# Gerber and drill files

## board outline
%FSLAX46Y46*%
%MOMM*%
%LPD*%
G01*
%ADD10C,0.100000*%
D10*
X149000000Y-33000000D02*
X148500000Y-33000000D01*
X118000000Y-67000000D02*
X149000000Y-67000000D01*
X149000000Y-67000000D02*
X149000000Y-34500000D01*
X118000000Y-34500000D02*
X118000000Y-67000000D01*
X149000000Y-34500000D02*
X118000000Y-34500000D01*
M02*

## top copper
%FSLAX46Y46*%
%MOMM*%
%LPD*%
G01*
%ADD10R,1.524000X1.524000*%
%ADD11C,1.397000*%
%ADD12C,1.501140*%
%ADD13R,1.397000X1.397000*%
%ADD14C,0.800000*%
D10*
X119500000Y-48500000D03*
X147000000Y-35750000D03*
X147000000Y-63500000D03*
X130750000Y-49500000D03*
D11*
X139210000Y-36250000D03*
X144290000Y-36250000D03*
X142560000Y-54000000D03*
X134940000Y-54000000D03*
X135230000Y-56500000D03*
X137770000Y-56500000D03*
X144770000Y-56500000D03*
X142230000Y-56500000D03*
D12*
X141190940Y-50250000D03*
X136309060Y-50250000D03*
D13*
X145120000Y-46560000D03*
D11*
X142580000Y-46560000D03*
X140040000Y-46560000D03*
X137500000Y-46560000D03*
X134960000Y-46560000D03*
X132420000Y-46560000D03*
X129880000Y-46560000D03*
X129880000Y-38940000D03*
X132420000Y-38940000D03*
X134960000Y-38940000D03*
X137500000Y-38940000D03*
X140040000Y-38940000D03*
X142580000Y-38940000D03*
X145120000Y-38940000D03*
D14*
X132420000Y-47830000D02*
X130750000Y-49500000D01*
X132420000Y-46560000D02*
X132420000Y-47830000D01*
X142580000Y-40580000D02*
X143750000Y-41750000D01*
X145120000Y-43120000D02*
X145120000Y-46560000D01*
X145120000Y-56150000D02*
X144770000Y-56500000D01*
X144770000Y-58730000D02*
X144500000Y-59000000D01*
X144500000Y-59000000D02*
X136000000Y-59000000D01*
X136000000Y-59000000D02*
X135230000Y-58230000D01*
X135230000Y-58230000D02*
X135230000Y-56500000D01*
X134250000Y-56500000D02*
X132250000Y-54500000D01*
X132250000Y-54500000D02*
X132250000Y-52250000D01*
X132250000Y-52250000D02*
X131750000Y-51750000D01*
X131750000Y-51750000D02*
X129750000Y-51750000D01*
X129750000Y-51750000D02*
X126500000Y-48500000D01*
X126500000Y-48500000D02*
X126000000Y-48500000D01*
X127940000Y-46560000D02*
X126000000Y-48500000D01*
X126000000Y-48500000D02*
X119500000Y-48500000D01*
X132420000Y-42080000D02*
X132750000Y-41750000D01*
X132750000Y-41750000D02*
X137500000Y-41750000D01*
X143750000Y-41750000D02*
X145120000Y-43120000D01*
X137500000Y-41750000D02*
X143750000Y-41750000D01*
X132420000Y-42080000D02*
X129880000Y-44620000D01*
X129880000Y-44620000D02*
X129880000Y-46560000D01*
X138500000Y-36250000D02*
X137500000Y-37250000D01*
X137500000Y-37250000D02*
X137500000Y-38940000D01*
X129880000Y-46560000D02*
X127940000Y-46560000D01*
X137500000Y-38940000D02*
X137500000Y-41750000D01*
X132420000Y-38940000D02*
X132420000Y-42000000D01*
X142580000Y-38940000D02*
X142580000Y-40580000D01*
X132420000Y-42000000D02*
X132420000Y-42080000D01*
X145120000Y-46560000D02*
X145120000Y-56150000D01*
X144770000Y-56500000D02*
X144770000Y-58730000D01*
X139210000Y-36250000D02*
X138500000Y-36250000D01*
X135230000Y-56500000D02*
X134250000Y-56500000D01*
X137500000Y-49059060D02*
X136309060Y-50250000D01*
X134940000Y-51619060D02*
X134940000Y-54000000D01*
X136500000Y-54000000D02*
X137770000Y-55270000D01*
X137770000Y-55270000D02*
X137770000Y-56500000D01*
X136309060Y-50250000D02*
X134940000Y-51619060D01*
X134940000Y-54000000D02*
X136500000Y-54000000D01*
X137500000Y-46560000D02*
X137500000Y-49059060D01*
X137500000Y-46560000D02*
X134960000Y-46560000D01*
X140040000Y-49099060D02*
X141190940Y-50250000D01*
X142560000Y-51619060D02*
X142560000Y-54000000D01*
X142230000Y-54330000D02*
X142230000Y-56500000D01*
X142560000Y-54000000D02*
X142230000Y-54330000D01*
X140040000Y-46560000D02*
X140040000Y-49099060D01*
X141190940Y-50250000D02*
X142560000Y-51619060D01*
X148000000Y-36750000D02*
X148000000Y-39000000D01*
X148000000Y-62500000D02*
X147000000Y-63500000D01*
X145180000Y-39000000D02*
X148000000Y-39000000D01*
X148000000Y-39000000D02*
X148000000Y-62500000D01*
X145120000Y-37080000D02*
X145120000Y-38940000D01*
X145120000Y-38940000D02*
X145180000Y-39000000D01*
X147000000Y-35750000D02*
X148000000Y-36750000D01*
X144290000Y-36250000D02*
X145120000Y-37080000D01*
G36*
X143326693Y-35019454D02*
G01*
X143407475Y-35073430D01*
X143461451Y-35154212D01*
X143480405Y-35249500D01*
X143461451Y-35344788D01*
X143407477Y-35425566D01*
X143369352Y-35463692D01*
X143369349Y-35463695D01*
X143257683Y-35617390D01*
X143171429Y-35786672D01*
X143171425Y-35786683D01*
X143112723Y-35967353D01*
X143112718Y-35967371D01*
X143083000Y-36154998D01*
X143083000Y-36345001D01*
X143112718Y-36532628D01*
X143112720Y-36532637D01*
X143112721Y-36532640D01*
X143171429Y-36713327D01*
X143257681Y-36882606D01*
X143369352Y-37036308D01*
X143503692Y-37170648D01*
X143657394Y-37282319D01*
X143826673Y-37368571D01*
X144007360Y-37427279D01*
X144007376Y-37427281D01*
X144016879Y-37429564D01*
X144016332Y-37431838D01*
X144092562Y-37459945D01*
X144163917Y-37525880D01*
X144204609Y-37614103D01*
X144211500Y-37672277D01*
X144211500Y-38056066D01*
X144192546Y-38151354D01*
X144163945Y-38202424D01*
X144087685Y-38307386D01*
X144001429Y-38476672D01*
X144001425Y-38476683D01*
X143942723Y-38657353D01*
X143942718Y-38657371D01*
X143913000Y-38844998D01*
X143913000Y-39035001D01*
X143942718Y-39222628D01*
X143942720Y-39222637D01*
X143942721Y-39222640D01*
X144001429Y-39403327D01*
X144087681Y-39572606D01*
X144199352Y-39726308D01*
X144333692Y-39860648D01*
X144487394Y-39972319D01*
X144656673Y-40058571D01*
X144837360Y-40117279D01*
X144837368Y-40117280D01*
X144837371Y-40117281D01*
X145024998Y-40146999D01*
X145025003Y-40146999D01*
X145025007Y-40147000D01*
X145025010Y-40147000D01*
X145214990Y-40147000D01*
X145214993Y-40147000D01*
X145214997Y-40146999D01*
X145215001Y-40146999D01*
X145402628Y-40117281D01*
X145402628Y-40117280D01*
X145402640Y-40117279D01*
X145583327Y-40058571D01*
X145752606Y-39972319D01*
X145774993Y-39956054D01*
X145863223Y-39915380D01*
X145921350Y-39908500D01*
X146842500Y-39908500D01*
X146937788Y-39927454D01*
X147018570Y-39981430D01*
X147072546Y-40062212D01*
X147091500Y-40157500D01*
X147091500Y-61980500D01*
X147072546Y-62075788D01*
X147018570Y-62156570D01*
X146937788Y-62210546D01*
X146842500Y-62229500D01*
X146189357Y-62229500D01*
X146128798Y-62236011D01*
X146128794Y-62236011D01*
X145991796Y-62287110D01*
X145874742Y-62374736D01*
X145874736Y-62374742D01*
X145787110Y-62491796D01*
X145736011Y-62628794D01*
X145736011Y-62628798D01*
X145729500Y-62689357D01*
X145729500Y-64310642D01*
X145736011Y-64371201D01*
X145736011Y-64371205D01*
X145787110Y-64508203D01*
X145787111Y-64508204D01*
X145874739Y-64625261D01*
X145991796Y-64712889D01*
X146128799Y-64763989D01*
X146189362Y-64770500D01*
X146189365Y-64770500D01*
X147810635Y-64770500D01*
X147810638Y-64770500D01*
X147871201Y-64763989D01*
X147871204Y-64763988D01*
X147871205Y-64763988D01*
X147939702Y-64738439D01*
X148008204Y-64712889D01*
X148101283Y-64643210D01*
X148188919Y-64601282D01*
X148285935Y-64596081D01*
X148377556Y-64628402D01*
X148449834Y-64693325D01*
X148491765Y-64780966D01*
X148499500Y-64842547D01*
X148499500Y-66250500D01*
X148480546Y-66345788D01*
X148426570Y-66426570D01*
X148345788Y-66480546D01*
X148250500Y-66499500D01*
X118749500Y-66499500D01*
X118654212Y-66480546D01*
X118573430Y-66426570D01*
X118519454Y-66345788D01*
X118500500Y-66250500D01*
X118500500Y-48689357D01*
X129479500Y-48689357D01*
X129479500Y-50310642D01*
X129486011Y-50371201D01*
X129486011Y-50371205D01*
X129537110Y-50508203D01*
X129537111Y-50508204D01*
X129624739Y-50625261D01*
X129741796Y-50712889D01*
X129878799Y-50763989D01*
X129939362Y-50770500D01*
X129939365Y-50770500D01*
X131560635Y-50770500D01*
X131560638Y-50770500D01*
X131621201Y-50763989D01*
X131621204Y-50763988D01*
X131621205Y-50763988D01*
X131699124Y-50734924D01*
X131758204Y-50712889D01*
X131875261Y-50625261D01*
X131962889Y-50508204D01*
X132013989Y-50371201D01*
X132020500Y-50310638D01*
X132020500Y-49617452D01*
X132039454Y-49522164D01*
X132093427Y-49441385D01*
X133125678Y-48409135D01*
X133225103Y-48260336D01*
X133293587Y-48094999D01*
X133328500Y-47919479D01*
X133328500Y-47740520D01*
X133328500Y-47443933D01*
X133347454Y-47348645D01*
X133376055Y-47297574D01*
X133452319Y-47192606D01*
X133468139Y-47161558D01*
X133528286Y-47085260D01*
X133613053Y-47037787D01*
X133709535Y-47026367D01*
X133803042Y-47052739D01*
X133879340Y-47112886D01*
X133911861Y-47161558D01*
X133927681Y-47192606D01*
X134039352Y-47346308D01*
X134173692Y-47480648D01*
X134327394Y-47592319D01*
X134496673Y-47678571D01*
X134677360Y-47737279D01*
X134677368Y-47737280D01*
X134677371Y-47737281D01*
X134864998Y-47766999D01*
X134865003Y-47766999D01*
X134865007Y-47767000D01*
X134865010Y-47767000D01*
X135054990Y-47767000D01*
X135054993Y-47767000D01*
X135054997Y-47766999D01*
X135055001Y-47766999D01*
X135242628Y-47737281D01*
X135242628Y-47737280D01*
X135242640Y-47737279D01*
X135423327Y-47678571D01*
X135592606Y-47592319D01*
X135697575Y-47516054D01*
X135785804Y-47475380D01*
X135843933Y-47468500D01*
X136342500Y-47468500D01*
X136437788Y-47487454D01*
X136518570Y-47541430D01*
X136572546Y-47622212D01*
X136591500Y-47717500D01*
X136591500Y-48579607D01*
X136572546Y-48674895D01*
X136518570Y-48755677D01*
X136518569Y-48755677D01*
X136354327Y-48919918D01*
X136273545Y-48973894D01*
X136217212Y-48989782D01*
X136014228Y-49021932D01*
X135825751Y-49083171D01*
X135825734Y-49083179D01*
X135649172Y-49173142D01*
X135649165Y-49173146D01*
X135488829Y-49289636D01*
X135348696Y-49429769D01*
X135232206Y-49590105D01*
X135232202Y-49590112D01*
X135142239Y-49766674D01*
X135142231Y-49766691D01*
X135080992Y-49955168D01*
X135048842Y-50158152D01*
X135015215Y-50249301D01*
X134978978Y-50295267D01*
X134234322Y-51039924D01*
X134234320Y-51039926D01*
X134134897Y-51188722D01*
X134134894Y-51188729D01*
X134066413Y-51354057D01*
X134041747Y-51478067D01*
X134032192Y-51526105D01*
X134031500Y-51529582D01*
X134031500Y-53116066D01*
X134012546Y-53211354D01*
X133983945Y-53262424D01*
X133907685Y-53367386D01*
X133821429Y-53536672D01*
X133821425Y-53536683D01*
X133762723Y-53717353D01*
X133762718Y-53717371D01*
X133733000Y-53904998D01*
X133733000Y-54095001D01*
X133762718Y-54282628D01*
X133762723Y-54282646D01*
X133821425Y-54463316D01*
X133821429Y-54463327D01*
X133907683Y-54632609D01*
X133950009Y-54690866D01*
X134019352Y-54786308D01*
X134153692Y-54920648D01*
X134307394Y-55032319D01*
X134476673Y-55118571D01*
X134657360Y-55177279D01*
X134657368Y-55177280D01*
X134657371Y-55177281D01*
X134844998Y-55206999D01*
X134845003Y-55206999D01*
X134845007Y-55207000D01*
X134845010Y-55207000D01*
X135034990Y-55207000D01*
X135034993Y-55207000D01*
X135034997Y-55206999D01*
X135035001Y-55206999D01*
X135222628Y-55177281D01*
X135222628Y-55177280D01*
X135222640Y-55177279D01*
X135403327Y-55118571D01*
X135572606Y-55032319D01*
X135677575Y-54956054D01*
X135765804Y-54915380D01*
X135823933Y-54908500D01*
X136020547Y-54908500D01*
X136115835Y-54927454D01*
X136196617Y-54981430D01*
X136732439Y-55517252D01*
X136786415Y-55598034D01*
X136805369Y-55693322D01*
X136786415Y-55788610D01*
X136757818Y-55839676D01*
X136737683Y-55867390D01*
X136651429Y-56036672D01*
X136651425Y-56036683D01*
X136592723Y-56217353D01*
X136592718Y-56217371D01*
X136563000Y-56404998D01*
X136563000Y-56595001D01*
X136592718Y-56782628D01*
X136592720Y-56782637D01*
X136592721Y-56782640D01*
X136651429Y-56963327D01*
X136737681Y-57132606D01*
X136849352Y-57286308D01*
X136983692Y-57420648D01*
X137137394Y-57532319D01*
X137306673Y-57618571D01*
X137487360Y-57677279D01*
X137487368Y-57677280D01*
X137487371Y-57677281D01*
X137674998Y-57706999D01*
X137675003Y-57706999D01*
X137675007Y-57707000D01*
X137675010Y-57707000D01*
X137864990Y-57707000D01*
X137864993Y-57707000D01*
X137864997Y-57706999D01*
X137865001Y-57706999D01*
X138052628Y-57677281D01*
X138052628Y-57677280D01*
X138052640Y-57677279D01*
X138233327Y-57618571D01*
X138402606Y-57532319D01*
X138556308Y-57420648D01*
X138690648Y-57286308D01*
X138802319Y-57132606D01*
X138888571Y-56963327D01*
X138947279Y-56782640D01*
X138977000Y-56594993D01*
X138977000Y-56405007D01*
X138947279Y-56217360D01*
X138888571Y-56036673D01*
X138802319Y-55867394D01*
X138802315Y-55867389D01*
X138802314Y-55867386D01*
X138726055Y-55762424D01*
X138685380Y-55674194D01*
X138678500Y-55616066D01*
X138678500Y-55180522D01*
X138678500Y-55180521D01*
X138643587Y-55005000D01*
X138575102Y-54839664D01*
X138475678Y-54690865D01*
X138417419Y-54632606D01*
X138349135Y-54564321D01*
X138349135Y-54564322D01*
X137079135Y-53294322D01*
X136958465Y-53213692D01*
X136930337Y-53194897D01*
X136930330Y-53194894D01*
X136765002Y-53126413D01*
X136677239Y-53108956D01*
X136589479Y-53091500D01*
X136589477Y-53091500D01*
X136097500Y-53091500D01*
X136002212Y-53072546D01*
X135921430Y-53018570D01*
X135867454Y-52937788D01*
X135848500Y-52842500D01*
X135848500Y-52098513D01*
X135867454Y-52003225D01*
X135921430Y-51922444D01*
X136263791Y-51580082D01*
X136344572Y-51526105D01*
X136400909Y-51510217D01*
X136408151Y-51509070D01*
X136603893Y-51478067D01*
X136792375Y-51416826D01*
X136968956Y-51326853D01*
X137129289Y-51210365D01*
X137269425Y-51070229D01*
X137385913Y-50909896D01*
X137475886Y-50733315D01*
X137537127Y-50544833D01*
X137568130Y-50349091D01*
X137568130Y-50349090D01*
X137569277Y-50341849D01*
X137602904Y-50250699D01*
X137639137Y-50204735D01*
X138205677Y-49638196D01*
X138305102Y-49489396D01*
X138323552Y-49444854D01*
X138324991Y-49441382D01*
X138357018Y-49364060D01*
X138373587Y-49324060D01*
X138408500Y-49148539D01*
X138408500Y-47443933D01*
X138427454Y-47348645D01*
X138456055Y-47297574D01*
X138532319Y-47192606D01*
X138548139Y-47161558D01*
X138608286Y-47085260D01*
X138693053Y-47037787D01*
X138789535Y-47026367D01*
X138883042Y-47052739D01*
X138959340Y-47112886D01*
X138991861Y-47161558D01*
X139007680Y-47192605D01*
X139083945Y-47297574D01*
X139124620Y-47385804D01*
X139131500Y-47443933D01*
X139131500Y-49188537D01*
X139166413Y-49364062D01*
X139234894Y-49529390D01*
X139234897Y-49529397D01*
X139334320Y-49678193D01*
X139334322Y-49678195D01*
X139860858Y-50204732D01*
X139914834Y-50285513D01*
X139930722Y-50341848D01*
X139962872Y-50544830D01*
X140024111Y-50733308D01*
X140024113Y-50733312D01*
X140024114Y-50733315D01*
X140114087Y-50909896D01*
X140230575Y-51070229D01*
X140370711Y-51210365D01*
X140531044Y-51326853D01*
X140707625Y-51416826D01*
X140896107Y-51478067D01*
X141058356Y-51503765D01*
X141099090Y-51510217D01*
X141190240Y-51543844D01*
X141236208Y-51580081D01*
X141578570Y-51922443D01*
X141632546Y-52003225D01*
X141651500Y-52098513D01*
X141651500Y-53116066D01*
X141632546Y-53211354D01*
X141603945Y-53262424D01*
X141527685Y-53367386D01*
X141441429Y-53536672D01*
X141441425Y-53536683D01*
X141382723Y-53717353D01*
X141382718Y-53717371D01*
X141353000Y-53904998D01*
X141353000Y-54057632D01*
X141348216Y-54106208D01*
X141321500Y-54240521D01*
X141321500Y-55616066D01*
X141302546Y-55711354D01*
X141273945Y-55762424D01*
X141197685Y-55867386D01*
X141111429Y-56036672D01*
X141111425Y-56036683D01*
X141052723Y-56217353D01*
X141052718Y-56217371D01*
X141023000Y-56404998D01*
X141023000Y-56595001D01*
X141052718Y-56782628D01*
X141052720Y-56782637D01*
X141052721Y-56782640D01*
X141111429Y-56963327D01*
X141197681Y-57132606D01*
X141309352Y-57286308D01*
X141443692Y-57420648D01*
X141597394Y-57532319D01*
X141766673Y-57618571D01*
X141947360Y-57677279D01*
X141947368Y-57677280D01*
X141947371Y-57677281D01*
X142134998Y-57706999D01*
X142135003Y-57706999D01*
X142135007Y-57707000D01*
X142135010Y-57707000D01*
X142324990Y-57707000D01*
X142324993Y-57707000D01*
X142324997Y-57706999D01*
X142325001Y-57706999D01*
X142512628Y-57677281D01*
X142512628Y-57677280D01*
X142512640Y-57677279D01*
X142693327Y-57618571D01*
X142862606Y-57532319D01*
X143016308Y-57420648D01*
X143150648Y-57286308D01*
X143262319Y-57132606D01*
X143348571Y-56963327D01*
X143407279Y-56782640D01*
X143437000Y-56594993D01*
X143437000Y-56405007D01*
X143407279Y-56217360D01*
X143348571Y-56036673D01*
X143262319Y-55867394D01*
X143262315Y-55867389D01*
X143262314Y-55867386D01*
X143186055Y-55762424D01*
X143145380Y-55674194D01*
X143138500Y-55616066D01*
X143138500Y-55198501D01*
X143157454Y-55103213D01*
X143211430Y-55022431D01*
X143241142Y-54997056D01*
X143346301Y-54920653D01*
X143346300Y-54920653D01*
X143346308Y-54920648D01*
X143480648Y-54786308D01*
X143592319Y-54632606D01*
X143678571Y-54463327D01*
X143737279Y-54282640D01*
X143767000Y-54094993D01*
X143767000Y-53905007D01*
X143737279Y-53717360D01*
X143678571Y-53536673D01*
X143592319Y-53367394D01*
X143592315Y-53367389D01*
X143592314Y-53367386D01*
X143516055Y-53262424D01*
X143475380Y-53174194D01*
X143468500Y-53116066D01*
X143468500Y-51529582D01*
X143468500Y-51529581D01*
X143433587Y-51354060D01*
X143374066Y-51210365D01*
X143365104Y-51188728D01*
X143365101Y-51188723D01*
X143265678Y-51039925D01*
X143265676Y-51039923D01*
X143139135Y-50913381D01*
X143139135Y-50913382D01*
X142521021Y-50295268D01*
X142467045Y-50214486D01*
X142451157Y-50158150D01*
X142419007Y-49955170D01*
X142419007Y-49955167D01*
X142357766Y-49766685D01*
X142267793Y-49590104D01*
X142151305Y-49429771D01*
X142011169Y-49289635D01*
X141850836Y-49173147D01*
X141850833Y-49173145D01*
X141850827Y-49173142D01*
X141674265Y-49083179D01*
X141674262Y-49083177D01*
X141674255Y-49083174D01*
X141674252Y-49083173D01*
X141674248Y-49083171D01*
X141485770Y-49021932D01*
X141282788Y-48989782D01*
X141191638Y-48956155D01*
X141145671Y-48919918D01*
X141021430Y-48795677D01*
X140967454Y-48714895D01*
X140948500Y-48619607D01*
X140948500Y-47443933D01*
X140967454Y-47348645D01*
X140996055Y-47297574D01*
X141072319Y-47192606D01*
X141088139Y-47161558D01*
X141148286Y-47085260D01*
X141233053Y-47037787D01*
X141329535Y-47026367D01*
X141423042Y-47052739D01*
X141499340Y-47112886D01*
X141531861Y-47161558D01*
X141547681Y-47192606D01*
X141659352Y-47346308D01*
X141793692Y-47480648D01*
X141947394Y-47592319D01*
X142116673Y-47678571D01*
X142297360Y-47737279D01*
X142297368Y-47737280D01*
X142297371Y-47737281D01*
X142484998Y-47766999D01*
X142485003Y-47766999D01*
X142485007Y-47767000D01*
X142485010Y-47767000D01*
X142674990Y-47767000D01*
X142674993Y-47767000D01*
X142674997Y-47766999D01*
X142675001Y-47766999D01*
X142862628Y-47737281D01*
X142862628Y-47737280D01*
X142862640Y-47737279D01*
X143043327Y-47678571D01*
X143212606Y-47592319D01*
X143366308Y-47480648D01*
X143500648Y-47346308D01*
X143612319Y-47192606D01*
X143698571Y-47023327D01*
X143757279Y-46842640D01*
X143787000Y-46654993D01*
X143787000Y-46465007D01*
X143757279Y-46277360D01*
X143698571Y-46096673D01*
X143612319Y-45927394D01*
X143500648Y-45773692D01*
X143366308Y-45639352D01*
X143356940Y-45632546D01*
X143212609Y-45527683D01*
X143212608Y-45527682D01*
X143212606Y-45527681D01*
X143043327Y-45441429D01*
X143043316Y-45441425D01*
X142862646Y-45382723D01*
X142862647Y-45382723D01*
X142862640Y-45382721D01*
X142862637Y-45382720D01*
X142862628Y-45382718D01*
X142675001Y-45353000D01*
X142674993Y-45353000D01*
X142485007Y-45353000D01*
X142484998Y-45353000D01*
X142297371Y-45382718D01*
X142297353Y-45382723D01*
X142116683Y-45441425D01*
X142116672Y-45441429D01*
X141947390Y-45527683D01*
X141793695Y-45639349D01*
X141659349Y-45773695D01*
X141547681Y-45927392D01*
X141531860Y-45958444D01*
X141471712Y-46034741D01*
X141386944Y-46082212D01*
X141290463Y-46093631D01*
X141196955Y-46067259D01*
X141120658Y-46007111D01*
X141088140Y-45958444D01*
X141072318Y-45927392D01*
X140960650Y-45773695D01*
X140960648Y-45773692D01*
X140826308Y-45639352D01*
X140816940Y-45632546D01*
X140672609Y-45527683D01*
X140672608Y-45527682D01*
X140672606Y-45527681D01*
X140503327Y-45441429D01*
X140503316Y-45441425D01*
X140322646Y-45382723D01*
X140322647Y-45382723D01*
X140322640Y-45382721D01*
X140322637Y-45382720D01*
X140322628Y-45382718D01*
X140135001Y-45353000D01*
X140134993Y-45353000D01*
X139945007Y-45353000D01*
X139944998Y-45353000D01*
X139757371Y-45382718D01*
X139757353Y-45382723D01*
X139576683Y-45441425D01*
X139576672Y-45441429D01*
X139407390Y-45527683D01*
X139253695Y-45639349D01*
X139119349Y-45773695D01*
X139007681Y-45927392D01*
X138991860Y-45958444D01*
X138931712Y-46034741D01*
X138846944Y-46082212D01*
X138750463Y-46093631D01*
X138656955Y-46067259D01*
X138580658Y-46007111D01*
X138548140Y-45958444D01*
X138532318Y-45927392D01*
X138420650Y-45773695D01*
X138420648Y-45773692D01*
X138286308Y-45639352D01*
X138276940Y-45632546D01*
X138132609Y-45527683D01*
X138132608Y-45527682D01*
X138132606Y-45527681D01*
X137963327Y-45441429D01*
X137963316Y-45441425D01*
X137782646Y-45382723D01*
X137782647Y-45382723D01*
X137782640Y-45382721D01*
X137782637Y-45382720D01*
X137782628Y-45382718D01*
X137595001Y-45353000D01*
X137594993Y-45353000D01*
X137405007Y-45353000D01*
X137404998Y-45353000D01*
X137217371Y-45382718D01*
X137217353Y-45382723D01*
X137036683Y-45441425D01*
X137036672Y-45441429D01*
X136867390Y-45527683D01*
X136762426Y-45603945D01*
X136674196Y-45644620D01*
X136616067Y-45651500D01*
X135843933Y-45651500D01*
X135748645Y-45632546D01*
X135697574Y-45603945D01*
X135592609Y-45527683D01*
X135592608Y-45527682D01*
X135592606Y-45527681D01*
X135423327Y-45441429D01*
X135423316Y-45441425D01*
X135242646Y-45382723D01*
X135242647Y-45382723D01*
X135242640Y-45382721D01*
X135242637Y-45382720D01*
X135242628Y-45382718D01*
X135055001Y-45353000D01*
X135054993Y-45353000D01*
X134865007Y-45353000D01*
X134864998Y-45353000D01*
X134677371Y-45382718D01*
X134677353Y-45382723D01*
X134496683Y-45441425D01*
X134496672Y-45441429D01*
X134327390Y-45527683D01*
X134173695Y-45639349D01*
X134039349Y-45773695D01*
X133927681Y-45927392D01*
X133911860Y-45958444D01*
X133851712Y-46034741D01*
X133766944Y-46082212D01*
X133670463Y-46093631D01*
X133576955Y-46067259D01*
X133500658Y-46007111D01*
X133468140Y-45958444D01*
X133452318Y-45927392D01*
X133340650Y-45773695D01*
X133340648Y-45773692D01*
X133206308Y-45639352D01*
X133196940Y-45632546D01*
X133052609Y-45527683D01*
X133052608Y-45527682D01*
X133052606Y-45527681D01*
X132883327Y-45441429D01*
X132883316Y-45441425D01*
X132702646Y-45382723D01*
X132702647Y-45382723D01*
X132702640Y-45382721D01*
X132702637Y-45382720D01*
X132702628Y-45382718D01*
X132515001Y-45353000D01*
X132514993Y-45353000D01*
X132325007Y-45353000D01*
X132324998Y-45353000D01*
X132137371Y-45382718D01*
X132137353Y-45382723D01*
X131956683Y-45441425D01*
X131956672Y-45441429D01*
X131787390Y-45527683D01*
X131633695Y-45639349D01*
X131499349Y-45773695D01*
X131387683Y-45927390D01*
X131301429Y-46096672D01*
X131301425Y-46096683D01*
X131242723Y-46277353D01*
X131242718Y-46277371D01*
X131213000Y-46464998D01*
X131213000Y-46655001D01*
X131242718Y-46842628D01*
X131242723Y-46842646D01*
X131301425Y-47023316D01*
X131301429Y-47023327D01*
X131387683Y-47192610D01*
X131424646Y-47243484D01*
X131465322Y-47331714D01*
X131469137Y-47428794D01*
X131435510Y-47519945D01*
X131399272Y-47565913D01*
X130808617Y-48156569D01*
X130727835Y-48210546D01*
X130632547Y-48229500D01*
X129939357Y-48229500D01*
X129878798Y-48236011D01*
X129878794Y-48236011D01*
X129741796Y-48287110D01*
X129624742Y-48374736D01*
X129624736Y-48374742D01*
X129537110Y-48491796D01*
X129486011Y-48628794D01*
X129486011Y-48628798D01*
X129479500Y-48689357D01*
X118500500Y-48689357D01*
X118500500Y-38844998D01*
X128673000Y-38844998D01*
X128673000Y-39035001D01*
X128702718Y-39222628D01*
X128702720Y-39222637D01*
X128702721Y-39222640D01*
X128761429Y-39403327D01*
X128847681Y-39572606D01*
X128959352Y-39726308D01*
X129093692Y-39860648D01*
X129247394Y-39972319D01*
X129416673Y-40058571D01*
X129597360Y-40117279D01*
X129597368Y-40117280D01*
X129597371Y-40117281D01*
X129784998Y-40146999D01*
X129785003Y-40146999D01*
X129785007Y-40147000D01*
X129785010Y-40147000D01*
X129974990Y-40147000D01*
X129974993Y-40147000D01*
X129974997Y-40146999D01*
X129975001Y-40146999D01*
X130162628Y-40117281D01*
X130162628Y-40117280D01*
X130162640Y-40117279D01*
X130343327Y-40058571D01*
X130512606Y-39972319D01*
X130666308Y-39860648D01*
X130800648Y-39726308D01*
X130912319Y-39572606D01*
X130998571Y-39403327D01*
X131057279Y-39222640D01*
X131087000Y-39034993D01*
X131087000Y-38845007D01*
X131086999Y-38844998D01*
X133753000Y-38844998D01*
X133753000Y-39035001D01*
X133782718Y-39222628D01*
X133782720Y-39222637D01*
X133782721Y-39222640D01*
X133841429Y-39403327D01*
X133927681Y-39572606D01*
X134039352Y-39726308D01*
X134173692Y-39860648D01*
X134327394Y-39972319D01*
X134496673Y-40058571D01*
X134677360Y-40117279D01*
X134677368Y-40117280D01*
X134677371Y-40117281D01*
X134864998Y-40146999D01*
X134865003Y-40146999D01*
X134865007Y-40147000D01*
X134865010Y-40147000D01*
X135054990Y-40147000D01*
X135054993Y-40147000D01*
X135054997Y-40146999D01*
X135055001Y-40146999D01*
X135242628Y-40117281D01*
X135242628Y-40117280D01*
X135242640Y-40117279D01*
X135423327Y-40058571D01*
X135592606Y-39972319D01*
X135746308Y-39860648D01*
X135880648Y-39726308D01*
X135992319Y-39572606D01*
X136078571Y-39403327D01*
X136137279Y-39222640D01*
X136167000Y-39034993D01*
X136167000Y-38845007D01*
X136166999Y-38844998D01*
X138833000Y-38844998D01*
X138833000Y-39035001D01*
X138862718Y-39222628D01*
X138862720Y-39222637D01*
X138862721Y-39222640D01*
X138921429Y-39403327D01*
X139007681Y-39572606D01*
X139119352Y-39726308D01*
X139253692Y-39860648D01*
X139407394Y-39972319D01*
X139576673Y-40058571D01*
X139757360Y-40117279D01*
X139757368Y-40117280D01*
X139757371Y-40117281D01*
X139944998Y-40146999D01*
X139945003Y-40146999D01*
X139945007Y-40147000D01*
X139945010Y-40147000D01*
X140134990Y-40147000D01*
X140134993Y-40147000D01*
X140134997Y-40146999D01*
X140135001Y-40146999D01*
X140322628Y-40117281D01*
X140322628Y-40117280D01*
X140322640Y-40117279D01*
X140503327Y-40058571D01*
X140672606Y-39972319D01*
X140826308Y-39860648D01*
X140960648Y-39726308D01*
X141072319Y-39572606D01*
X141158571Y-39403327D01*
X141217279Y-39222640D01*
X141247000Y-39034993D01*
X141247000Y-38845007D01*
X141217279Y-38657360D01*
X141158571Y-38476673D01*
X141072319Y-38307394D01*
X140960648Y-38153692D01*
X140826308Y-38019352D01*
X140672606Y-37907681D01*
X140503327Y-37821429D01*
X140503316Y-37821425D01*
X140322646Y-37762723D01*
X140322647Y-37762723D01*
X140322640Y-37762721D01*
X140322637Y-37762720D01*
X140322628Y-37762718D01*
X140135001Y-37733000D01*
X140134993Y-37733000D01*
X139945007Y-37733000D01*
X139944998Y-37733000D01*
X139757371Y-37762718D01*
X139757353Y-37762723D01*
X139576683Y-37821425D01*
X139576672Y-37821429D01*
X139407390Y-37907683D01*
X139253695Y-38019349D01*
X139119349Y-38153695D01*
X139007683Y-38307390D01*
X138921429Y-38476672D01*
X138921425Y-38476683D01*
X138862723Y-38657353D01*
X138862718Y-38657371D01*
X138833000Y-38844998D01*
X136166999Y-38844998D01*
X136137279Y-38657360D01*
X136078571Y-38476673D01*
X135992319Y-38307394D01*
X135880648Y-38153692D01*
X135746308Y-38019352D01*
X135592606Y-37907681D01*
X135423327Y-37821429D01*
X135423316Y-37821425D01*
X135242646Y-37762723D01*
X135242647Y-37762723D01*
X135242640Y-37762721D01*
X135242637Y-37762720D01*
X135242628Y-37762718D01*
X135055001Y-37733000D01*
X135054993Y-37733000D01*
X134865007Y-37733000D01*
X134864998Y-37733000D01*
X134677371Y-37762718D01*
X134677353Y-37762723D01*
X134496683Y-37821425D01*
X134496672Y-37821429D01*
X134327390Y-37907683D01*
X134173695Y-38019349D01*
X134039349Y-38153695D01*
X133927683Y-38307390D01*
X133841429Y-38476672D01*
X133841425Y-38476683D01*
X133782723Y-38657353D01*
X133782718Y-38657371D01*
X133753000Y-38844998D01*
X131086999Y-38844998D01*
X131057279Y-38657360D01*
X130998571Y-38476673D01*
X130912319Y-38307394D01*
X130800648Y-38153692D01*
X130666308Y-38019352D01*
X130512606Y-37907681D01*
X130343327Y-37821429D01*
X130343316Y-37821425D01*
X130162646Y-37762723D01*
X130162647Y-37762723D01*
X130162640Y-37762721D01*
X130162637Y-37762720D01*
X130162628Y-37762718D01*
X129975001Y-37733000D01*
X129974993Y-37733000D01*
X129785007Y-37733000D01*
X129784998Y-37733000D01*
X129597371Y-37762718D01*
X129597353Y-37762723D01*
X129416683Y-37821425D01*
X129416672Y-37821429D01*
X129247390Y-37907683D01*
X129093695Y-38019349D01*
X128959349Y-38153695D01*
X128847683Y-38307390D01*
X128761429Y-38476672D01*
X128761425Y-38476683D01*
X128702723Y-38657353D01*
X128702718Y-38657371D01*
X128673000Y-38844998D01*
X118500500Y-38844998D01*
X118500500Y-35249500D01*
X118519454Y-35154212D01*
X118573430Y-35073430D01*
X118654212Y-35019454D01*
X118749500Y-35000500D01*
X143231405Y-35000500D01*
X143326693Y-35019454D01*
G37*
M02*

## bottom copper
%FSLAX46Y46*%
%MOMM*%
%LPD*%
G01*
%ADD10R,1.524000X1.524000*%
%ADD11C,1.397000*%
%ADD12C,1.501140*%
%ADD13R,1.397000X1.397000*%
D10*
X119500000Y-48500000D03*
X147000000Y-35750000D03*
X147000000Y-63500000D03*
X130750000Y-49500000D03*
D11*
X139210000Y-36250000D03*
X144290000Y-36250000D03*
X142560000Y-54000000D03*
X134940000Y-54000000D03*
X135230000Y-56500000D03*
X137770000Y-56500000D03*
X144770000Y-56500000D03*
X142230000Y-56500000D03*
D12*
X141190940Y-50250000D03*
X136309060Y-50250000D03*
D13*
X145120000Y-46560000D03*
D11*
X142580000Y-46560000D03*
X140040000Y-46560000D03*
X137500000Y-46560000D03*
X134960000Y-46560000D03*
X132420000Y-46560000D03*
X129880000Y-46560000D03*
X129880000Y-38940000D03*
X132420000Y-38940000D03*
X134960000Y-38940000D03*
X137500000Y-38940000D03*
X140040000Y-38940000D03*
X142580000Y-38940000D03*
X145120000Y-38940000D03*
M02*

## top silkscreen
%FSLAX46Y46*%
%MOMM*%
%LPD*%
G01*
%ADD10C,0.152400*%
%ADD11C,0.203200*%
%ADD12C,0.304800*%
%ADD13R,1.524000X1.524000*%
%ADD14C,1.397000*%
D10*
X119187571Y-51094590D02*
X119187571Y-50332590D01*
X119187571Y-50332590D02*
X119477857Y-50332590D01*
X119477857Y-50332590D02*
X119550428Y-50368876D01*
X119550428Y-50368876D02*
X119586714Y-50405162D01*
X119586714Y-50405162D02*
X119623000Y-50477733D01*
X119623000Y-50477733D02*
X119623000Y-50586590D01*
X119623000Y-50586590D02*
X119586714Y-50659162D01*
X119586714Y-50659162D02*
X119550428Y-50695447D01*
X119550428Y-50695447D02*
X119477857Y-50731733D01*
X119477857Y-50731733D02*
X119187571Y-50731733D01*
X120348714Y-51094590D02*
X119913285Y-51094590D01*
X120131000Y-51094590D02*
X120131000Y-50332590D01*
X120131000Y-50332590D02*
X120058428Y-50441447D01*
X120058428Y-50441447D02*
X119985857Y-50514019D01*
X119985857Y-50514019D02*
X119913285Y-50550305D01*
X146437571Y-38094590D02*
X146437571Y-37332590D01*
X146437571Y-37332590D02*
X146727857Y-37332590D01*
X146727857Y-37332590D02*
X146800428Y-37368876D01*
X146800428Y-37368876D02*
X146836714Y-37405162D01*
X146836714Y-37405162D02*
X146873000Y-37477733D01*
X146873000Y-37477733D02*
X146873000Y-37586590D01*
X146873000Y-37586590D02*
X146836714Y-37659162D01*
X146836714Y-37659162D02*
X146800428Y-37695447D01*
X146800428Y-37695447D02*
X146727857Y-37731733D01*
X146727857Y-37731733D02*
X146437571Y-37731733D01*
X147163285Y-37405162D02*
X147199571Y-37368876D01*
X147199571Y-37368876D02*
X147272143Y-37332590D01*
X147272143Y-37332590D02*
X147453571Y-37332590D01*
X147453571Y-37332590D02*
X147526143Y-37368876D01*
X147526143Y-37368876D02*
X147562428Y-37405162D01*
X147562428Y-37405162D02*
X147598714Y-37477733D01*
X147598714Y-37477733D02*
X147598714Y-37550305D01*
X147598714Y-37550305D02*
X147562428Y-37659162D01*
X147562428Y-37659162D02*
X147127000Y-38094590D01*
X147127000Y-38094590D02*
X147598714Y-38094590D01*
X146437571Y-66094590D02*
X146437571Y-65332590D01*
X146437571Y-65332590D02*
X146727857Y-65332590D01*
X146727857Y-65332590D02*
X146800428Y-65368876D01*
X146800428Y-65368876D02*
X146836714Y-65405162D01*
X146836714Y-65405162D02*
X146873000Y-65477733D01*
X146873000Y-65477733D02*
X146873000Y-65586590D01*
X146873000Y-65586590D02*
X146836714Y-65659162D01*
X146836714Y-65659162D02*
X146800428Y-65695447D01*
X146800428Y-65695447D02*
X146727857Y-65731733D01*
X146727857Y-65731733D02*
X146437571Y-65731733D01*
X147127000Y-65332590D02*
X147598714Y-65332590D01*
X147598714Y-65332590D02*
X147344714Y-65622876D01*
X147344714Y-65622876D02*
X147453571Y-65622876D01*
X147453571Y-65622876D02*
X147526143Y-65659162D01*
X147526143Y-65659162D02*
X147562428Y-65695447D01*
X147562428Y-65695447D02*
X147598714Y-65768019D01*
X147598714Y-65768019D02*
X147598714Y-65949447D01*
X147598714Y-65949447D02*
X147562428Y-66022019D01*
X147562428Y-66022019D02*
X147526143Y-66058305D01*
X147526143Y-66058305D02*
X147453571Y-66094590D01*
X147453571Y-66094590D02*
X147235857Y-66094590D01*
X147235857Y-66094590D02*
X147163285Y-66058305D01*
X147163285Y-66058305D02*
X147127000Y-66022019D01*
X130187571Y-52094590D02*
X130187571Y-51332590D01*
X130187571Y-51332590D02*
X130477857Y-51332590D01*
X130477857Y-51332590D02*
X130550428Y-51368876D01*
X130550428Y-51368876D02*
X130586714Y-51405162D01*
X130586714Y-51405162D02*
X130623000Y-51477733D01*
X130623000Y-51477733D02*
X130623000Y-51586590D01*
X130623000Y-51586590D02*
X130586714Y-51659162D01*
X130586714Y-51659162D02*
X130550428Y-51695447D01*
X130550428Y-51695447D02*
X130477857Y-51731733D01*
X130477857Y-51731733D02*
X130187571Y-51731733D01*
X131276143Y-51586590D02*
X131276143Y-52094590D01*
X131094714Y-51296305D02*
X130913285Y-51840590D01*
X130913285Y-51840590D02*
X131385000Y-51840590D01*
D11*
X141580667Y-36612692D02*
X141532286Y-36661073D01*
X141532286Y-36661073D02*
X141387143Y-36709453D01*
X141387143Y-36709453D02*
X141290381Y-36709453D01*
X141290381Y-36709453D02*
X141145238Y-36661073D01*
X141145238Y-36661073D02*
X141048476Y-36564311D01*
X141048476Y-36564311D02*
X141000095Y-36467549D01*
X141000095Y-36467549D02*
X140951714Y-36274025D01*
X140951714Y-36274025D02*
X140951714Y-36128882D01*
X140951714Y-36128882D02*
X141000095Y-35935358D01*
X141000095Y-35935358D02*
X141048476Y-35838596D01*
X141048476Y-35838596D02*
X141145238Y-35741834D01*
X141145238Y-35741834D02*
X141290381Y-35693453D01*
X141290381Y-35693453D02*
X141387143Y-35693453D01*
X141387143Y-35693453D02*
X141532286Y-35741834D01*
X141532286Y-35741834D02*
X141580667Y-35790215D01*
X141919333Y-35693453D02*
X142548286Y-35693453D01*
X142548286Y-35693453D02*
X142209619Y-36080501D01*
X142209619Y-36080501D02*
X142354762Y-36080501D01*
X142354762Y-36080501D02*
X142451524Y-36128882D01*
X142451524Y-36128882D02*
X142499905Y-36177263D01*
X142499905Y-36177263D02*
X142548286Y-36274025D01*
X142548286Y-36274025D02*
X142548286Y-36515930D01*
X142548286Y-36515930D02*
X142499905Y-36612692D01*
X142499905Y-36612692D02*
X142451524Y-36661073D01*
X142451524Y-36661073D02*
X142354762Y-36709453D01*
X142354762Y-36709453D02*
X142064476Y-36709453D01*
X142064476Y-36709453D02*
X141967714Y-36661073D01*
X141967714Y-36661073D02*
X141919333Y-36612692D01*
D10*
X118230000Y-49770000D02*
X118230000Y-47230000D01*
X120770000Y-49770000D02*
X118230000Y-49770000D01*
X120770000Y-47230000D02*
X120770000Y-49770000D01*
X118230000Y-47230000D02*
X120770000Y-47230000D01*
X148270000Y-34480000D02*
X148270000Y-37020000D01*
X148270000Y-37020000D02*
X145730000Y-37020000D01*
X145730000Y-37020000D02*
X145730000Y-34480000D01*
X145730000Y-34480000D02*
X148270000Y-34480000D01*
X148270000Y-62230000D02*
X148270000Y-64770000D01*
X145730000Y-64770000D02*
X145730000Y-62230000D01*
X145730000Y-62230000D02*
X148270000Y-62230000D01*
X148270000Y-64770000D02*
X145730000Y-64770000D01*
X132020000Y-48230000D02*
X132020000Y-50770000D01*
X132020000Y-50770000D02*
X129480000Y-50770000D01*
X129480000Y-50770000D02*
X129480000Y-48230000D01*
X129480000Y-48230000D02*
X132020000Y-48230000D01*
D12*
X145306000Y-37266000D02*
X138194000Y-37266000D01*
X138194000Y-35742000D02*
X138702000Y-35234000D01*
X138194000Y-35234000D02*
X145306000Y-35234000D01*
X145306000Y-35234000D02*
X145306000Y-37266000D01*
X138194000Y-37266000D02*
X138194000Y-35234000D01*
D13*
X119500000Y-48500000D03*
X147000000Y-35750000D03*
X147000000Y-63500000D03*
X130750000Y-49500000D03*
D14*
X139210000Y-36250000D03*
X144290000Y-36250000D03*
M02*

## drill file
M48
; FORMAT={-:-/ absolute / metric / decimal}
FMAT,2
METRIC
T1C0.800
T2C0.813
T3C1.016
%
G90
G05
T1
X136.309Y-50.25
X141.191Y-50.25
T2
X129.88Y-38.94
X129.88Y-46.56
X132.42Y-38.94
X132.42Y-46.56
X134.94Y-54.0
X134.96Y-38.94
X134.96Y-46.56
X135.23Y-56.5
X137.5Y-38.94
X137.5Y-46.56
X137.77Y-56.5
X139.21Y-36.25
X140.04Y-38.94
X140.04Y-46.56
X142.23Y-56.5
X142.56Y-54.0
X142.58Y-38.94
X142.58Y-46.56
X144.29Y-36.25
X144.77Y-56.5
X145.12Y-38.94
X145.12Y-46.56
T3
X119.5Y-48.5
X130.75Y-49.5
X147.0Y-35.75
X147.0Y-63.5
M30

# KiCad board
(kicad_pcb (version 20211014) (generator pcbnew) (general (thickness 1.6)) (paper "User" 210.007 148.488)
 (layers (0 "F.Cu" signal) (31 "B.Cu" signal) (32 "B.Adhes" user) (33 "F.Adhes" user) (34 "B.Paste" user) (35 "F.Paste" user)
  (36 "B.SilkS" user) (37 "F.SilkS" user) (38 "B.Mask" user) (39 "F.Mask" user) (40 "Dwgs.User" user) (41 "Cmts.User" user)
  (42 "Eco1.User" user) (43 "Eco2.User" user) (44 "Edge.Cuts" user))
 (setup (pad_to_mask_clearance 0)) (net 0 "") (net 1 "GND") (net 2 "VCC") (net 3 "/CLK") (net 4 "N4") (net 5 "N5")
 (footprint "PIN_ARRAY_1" (layer "F.Cu") (at 119.5 48.5)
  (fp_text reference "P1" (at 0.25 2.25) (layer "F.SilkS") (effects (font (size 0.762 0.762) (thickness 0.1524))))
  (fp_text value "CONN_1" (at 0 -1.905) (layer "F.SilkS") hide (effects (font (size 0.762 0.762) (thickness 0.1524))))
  (fp_line (start -1.27 1.27) (end -1.27 -1.27) (layer "F.SilkS") (width 0.1524))
  (fp_line (start 1.27 1.27) (end -1.27 1.27) (layer "F.SilkS") (width 0.1524))
  (fp_line (start 1.27 -1.27) (end 1.27 1.27) (layer "F.SilkS") (width 0.1524))
  (fp_line (start -1.27 -1.27) (end 1.27 -1.27) (layer "F.SilkS") (width 0.1524))
  (pad "1" thru_hole rect locked (at 0 0) (size 1.524 1.524) (drill 1.016) (layers *.Cu *.Mask "F.SilkS") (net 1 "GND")))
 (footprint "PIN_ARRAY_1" (layer "F.Cu") (at 147 35.75)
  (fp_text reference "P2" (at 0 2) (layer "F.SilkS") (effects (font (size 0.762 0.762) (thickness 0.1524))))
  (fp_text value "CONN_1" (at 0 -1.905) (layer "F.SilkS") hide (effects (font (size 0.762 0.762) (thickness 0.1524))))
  (fp_line (start 1.27 -1.27) (end 1.27 1.27) (layer "F.SilkS") (width 0.1524))
  (fp_line (start 1.27 1.27) (end -1.27 1.27) (layer "F.SilkS") (width 0.1524))
  (fp_line (start -1.27 1.27) (end -1.27 -1.27) (layer "F.SilkS") (width 0.1524))
  (fp_line (start -1.27 -1.27) (end 1.27 -1.27) (layer "F.SilkS") (width 0.1524))
  (pad "1" thru_hole rect locked (at 0 0) (size 1.524 1.524) (drill 1.016) (layers *.Cu *.Mask "F.SilkS") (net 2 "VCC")))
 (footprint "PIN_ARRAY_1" (layer "F.Cu") (at 147 63.5)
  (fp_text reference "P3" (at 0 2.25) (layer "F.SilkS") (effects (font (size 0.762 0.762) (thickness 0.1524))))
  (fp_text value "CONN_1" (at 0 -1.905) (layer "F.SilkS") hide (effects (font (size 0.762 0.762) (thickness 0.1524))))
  (fp_line (start 1.27 -1.27) (end 1.27 1.27) (layer "F.SilkS") (width 0.1524))
  (fp_line (start -1.27 1.27) (end -1.27 -1.27) (layer "F.SilkS") (width 0.1524))
  (fp_line (start -1.27 -1.27) (end 1.27 -1.27) (layer "F.SilkS") (width 0.1524))
  (fp_line (start 1.27 1.27) (end -1.27 1.27) (layer "F.SilkS") (width 0.1524))
  (pad "1" thru_hole rect locked (at 0 0) (size 1.524 1.524) (drill 1.016) (layers *.Cu *.Mask "F.SilkS") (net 2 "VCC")))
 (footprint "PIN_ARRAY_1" (layer "F.Cu") (at 130.75 49.5)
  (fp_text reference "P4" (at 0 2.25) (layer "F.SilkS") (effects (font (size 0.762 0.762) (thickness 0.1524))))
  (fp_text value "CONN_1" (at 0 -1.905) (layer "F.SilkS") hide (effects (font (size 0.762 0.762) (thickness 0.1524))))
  (fp_line (start 1.27 -1.27) (end 1.27 1.27) (layer "F.SilkS") (width 0.1524))
  (fp_line (start 1.27 1.27) (end -1.27 1.27) (layer "F.SilkS") (width 0.1524))
  (fp_line (start -1.27 1.27) (end -1.27 -1.27) (layer "F.SilkS") (width 0.1524))
  (fp_line (start -1.27 -1.27) (end 1.27 -1.27) (layer "F.SilkS") (width 0.1524))
  (pad "1" thru_hole rect locked (at 0 0) (size 1.524 1.524) (drill 1.016) (layers *.Cu *.Mask "F.SilkS") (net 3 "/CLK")))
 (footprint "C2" (layer "F.Cu") (at 141.75 36.25)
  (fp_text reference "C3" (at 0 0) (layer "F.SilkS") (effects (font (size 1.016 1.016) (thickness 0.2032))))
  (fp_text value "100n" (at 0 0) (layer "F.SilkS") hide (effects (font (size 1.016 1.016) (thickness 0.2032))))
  (fp_line (start 3.556 1.016) (end -3.556 1.016) (layer "F.SilkS") (width 0.3048))
  (fp_line (start -3.556 -0.508) (end -3.048 -1.016) (layer "F.SilkS") (width 0.3048))
  (fp_line (start -3.556 -1.016) (end 3.556 -1.016) (layer "F.SilkS") (width 0.3048))
  (fp_line (start 3.556 -1.016) (end 3.556 1.016) (layer "F.SilkS") (width 0.3048))
  (fp_line (start -3.556 1.016) (end -3.556 -1.016) (layer "F.SilkS") (width 0.3048))
  (pad "1" thru_hole circle locked (at -2.54 0) (size 1.397 1.397) (drill 0.8128) (layers *.Cu *.Mask "F.SilkS") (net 1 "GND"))
  (pad "2" thru_hole circle locked (at 2.54 0) (size 1.397 1.397) (drill 0.8128) (layers *.Cu *.Mask "F.SilkS") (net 2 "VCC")))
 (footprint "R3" (layer "B.Cu") (at 138.75 54 180) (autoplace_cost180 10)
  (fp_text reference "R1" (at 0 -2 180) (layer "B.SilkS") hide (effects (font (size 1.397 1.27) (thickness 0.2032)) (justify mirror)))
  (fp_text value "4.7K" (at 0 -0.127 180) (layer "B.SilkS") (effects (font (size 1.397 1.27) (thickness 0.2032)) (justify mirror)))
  (pad "1" thru_hole circle locked (at -3.81 0 180) (size 1.397 1.397) (drill 0.8128) (layers *.Cu *.Mask "B.SilkS") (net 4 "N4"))
  (pad "2" thru_hole circle locked (at 3.81 0 180) (size 1.397 1.397) (drill 0.8128) (layers *.Cu *.Mask "B.SilkS") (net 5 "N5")))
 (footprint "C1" (layer "B.Cu") (at 136.5 56.5)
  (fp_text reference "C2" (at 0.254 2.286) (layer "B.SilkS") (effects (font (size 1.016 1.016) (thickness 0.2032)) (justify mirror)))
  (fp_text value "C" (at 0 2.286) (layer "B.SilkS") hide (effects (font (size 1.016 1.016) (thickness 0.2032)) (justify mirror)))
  (pad "1" thru_hole circle locked (at -1.27 0) (size 1.397 1.397) (drill 0.8128) (layers *.Cu *.Mask "B.SilkS") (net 1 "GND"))
  (pad "2" thru_hole circle locked (at 1.27 0) (size 1.397 1.397) (drill 0.8128) (layers *.Cu *.Mask "B.SilkS") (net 5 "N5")))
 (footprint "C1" (layer "B.Cu") (at 143.5 56.5 180)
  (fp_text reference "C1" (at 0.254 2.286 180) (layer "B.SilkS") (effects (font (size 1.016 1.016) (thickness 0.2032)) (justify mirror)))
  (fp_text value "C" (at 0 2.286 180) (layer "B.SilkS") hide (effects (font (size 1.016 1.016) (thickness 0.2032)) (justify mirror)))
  (pad "1" thru_hole circle locked (at -1.27 0 180) (size 1.397 1.397) (drill 0.8128) (layers *.Cu *.Mask "B.SilkS") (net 1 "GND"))
  (pad "2" thru_hole circle locked (at 1.27 0 180) (size 1.397 1.397) (drill 0.8128) (layers *.Cu *.Mask "B.SilkS") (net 4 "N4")))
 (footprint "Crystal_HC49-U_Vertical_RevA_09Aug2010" (layer "B.Cu") (at 138.75 50.25 180)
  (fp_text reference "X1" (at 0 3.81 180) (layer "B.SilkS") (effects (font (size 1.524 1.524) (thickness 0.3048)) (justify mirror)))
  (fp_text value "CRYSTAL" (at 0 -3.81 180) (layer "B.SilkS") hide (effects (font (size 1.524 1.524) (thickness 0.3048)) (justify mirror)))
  (pad "1" thru_hole circle locked (at -2.44094 0 180) (size 1.50114 1.50114) (drill 0.8001) (layers *.Cu *.Mask "B.SilkS") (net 4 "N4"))
  (pad "2" thru_hole circle locked (at 2.44094 0 180) (size 1.50114 1.50114) (drill 0.8001) (layers *.Cu *.Mask "B.SilkS") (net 5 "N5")))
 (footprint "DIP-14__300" (layer "B.Cu") (at 137.5 42.75 180)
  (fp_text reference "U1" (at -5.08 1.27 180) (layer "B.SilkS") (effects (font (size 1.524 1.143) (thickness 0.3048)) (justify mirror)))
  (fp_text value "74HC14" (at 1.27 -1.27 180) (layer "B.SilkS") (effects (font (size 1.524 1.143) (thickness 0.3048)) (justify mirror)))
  (pad "1" thru_hole rect locked (at -7.62 -3.81 180) (size 1.397 1.397) (drill 0.8128) (layers *.Cu *.Mask "B.SilkS") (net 1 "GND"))
  (pad "2" thru_hole circle locked (at -5.08 -3.81 180) (size 1.397 1.397) (drill 0.8128) (layers *.Cu *.Mask "B.SilkS"))
  (pad "3" thru_hole circle locked (at -2.54 -3.81 180) (size 1.397 1.397) (drill 0.8128) (layers *.Cu *.Mask "B.SilkS") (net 4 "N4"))
  (pad "4" thru_hole circle locked (at 0 -3.81 180) (size 1.397 1.397) (drill 0.8128) (layers *.Cu *.Mask "B.SilkS") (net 5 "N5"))
  (pad "5" thru_hole circle locked (at 2.54 -3.81 180) (size 1.397 1.397) (drill 0.8128) (layers *.Cu *.Mask "B.SilkS") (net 5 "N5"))
  (pad "6" thru_hole circle locked (at 5.08 -3.81 180) (size 1.397 1.397) (drill 0.8128) (layers *.Cu *.Mask "B.SilkS") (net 3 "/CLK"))
  (pad "7" thru_hole circle locked (at 7.62 -3.81 180) (size 1.397 1.397) (drill 0.8128) (layers *.Cu *.Mask "B.SilkS") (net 1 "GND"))
  (pad "8" thru_hole circle locked (at 7.62 3.81 180) (size 1.397 1.397) (drill 0.8128) (layers *.Cu *.Mask "B.SilkS"))
  (pad "9" thru_hole circle locked (at 5.08 3.81 180) (size 1.397 1.397) (drill 0.8128) (layers *.Cu *.Mask "B.SilkS") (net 1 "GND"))
  (pad "10" thru_hole circle locked (at 2.54 3.81 180) (size 1.397 1.397) (drill 0.8128) (layers *.Cu *.Mask "B.SilkS"))
  (pad "11" thru_hole circle locked (at 0 3.81 180) (size 1.397 1.397) (drill 0.8128) (layers *.Cu *.Mask "B.SilkS") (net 1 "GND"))
  (pad "12" thru_hole circle locked (at -2.54 3.81 180) (size 1.397 1.397) (drill 0.8128) (layers *.Cu *.Mask "B.SilkS"))
  (pad "13" thru_hole circle locked (at -5.08 3.81 180) (size 1.397 1.397) (drill 0.8128) (layers *.Cu *.Mask "B.SilkS") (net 1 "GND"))
  (pad "14" thru_hole circle locked (at -7.62 3.81 180) (size 1.397 1.397) (drill 0.8128) (layers *.Cu *.Mask "B.SilkS") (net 2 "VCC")))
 (gr_line (start 149 33) (end 148.5 33) (layer "Edge.Cuts") (width 0.1))
 (gr_line (start 118 67) (end 149 67) (layer "Edge.Cuts") (width 0.1))
 (gr_line (start 149 67) (end 149 34.5) (layer "Edge.Cuts") (width 0.1))
 (gr_line (start 118 34.5) (end 118 67) (layer "Edge.Cuts") (width 0.1))
 (gr_line (start 149 34.5) (end 118 34.5) (layer "Edge.Cuts") (width 0.1))
 (segment (start 132.42 47.83) (end 130.75 49.5) (width 0.8) (layer "F.Cu") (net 3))
 (segment (start 132.42 46.56) (end 132.42 47.83) (width 0.8) (layer "F.Cu") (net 3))
 (segment (start 142.58 40.58) (end 143.75 41.75) (width 0.8) (layer "F.Cu") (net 1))
 (segment (start 145.12 43.12) (end 145.12 46.56) (width 0.8) (layer "F.Cu") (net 1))
 (segment (start 145.12 56.15) (end 144.77 56.5) (width 0.8) (layer "F.Cu") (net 1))
 (segment (start 144.77 58.73) (end 144.5 59) (width 0.8) (layer "F.Cu") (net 1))
 (segment (start 144.5 59) (end 136 59) (width 0.8) (layer "F.Cu") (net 1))
 (segment (start 136 59) (end 135.23 58.23) (width 0.8) (layer "F.Cu") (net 1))
 (segment (start 135.23 58.23) (end 135.23 56.5) (width 0.8) (layer "F.Cu") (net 1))
 (segment (start 134.25 56.5) (end 132.25 54.5) (width 0.8) (layer "F.Cu") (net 1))
 (segment (start 132.25 54.5) (end 132.25 52.25) (width 0.8) (layer "F.Cu") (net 1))
 (segment (start 132.25 52.25) (end 131.75 51.75) (width 0.8) (layer "F.Cu") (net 1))
 (segment (start 131.75 51.75) (end 129.75 51.75) (width 0.8) (layer "F.Cu") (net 1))
 (segment (start 129.75 51.75) (end 126.5 48.5) (width 0.8) (layer "F.Cu") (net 1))
 (segment (start 126.5 48.5) (end 126 48.5) (width 0.8) (layer "F.Cu") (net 1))
 (segment (start 127.94 46.56) (end 126 48.5) (width 0.8) (layer "F.Cu") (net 1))
 (segment (start 126 48.5) (end 119.5 48.5) (width 0.8) (layer "F.Cu") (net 1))
 (segment (start 132.42 42.08) (end 132.75 41.75) (width 0.8) (layer "F.Cu") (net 1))
 (segment (start 132.75 41.75) (end 137.5 41.75) (width 0.8) (layer "F.Cu") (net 1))
 (segment (start 143.75 41.75) (end 145.12 43.12) (width 0.8) (layer "F.Cu") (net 1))
 (segment (start 137.5 41.75) (end 143.75 41.75) (width 0.8) (layer "F.Cu") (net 1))
 (segment (start 132.42 42.08) (end 129.88 44.62) (width 0.8) (layer "F.Cu") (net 1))
 (segment (start 129.88 44.62) (end 129.88 46.56) (width 0.8) (layer "F.Cu") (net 1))
 (segment (start 138.5 36.25) (end 137.5 37.25) (width 0.8) (layer "F.Cu") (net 1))
 (segment (start 137.5 37.25) (end 137.5 38.94) (width 0.8) (layer "F.Cu") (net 1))
 (segment (start 129.88 46.56) (end 127.94 46.56) (width 0.8) (layer "F.Cu") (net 1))
 (segment (start 137.5 38.94) (end 137.5 41.75) (width 0.8) (layer "F.Cu") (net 1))
 (segment (start 132.42 38.94) (end 132.42 42) (width 0.8) (layer "F.Cu") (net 1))
 (segment (start 142.58 38.94) (end 142.58 40.58) (width 0.8) (layer "F.Cu") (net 1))
 (segment (start 132.42 42) (end 132.42 42.08) (width 0.8) (layer "F.Cu") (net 1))
 (segment (start 145.12 46.56) (end 145.12 56.15) (width 0.8) (layer "F.Cu") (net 1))
 (segment (start 144.77 56.5) (end 144.77 58.73) (width 0.8) (layer "F.Cu") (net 1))
 (segment (start 139.21 36.25) (end 138.5 36.25) (width 0.8) (layer "F.Cu") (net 1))
 (segment (start 135.23 56.5) (end 134.25 56.5) (width 0.8) (layer "F.Cu") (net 1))
 (segment (start 137.5 49.05906) (end 136.30906 50.25) (width 0.8) (layer "F.Cu") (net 5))
 (segment (start 134.94 51.61906) (end 134.94 54) (width 0.8) (layer "F.Cu") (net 5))
 (segment (start 136.5 54) (end 137.77 55.27) (width 0.8) (layer "F.Cu") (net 5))
 (segment (start 137.77 55.27) (end 137.77 56.5) (width 0.8) (layer "F.Cu") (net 5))
 (segment (start 136.30906 50.25) (end 134.94 51.61906) (width 0.8) (layer "F.Cu") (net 5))
 (segment (start 134.94 54) (end 136.5 54) (width 0.8) (layer "F.Cu") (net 5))
 (segment (start 137.5 46.56) (end 137.5 49.05906) (width 0.8) (layer "F.Cu") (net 5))
 (segment (start 137.5 46.56) (end 134.96 46.56) (width 0.8) (layer "F.Cu") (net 5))
 (segment (start 140.04 49.09906) (end 141.19094 50.25) (width 0.8) (layer "F.Cu") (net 4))
 (segment (start 142.56 51.61906) (end 142.56 54) (width 0.8) (layer "F.Cu") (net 4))
 (segment (start 142.23 54.33) (end 142.23 56.5) (width 0.8) (layer "F.Cu") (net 4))
 (segment (start 142.56 54) (end 142.23 54.33) (width 0.8) (layer "F.Cu") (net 4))
 (segment (start 140.04 46.56) (end 140.04 49.09906) (width 0.8) (layer "F.Cu") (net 4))
 (segment (start 141.19094 50.25) (end 142.56 51.61906) (width 0.8) (layer "F.Cu") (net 4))
 (segment (start 148 36.75) (end 148 39) (width 0.8) (layer "F.Cu") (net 2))
 (segment (start 148 62.5) (end 147 63.5) (width 0.8) (layer "F.Cu") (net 2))
 (segment (start 145.18 39) (end 148 39) (width 0.8) (layer "F.Cu") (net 2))
 (segment (start 148 39) (end 148 62.5) (width 0.8) (layer "F.Cu") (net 2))
 (segment (start 145.12 37.08) (end 145.12 38.94) (width 0.8) (layer "F.Cu") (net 2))
 (segment (start 145.12 38.94) (end 145.18 39) (width 0.8) (layer "F.Cu") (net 2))
 (segment (start 147 35.75) (end 148 36.75) (width 0.8) (layer "F.Cu") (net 2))
 (segment (start 144.29 36.25) (end 145.12 37.08) (width 0.8) (layer "F.Cu") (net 2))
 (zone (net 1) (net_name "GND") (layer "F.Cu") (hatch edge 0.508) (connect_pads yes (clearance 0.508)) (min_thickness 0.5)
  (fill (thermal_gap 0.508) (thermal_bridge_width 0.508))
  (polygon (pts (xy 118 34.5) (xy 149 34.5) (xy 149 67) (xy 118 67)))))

